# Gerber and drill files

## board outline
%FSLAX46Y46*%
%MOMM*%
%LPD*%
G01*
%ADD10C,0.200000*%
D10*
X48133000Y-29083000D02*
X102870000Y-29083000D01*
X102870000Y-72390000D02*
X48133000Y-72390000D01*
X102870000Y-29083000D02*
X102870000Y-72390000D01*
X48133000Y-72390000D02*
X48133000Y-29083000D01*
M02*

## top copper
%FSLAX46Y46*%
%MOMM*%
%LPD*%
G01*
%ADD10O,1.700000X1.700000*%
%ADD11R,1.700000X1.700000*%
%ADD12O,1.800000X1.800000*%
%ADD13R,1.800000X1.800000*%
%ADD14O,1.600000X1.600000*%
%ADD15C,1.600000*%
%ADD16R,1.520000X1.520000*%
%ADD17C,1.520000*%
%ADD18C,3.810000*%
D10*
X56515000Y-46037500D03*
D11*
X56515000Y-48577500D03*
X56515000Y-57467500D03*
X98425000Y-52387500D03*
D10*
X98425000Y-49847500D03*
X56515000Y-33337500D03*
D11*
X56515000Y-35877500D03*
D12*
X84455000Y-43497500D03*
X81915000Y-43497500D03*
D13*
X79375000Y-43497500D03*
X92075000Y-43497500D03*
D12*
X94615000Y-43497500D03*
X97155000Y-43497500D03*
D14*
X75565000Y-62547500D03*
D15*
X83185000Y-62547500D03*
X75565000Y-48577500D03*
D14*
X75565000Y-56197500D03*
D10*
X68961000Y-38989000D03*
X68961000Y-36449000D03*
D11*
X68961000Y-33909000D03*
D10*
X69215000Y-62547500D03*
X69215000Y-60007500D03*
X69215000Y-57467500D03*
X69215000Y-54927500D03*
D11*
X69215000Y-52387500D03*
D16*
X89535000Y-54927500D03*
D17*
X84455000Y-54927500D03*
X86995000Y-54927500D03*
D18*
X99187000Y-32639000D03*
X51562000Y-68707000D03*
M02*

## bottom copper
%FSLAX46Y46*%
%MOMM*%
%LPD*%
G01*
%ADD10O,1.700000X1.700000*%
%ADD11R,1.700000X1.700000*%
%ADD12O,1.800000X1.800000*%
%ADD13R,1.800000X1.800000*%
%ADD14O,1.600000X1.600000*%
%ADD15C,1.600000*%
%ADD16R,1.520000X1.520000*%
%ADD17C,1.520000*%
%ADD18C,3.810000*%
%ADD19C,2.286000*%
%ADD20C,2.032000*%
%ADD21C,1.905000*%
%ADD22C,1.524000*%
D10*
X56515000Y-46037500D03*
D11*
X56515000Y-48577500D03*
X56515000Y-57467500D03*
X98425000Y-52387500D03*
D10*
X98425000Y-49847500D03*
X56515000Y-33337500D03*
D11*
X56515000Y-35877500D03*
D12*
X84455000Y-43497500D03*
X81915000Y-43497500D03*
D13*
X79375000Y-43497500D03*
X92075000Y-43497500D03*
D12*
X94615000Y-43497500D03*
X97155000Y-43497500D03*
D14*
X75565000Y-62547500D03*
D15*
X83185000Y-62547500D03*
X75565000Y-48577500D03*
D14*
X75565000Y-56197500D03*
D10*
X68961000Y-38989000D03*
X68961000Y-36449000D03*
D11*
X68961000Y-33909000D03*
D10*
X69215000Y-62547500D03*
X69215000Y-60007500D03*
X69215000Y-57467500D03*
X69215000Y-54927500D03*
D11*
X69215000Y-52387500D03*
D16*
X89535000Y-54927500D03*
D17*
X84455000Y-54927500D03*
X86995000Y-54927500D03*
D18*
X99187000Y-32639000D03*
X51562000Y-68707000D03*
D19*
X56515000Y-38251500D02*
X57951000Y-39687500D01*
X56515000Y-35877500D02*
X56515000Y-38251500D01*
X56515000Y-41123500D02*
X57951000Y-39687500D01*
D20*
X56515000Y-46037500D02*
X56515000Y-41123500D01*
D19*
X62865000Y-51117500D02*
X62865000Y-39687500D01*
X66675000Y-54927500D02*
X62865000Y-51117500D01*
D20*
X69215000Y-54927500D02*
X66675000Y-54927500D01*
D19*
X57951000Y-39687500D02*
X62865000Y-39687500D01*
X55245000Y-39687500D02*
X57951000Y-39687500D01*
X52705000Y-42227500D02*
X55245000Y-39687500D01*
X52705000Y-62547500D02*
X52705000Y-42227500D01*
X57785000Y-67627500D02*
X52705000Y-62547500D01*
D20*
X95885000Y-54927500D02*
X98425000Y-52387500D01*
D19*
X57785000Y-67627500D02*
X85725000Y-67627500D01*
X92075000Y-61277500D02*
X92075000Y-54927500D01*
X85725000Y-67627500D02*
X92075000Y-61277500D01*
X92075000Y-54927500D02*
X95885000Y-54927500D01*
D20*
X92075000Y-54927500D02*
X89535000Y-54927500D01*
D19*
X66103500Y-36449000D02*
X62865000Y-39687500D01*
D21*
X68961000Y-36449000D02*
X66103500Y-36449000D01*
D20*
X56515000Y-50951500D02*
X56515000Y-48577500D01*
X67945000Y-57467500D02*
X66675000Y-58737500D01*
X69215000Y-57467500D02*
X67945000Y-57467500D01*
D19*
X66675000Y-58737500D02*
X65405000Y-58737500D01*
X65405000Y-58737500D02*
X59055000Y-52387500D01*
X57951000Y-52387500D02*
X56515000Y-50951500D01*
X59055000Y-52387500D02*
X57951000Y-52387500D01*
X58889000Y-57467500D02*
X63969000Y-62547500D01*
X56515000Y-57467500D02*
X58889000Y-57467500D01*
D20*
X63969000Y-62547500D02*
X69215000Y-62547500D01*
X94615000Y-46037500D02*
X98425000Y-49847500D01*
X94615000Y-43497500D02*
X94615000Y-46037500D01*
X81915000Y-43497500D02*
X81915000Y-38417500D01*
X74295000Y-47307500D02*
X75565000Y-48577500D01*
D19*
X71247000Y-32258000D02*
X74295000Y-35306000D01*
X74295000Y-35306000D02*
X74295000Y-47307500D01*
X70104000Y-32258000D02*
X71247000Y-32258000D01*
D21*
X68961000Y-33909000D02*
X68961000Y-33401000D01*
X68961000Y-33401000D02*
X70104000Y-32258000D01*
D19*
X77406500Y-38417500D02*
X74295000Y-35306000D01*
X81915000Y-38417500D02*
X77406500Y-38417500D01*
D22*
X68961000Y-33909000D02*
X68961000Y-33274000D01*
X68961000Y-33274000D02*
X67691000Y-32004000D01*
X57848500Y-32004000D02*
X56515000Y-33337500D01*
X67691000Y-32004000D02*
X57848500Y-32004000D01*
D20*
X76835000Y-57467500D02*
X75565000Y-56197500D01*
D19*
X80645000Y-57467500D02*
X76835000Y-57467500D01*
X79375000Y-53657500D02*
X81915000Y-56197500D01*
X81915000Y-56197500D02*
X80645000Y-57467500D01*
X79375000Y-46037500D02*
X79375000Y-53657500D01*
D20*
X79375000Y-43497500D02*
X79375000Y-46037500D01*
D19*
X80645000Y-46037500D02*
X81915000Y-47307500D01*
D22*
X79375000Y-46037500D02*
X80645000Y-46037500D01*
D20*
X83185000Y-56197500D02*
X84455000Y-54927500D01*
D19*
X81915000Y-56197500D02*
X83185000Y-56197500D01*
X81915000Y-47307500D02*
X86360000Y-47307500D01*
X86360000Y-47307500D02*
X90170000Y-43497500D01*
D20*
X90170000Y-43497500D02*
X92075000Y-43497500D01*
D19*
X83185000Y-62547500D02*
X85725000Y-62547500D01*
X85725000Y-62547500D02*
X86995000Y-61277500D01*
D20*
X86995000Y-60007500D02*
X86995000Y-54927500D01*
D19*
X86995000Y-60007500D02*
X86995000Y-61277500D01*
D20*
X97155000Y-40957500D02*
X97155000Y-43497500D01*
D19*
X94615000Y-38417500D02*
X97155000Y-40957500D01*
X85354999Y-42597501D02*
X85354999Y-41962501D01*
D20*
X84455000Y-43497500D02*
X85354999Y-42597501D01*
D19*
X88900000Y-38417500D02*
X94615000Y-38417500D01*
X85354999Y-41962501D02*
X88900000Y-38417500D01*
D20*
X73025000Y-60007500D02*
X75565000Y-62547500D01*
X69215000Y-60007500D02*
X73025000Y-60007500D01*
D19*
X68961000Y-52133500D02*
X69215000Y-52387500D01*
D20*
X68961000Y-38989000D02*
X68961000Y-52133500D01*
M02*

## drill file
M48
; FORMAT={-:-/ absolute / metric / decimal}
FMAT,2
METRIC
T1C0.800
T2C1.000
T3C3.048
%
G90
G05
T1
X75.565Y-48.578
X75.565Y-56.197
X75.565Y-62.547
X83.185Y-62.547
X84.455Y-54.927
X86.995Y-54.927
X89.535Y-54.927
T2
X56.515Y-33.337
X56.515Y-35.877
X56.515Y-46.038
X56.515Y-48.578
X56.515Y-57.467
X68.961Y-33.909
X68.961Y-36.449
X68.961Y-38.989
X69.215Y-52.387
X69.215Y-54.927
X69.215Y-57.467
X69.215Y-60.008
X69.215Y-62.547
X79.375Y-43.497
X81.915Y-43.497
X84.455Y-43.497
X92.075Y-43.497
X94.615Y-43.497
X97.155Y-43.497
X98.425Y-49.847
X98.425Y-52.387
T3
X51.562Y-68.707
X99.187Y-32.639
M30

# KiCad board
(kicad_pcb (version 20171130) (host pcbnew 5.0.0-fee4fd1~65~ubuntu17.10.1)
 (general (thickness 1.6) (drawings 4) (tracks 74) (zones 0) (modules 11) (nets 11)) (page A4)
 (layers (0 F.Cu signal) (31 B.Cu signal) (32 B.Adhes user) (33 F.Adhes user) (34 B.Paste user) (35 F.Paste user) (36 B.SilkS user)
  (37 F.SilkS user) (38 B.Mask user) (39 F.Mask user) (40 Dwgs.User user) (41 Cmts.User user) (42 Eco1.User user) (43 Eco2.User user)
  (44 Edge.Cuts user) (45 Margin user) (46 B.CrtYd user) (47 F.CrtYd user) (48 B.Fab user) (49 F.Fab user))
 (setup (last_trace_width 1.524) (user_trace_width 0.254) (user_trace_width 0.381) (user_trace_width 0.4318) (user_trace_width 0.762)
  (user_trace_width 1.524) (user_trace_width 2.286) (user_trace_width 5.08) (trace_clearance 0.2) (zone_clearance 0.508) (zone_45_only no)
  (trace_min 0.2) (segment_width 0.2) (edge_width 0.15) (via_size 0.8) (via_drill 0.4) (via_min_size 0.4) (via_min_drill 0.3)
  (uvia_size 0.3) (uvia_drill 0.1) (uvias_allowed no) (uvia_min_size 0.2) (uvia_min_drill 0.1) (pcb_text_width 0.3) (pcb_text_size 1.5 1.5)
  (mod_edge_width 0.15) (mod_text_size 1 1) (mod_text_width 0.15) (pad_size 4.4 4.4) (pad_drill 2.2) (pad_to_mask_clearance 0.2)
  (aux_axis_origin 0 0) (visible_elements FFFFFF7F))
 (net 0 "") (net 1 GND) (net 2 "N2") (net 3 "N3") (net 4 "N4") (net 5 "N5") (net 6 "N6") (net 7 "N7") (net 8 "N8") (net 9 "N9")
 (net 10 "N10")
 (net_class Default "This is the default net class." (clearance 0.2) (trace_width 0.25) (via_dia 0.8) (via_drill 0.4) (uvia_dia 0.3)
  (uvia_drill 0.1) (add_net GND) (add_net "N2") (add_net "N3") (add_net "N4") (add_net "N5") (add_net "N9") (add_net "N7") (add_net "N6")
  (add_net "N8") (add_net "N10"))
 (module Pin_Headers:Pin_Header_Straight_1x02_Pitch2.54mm (layer F.Cu) (at 56.515 48.5775 180)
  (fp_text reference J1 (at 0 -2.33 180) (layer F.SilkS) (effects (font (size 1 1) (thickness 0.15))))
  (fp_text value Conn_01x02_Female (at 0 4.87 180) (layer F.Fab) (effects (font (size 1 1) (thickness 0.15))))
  (pad 2 thru_hole oval (at 0 2.54 180) (size 1.7 1.7) (drill 1) (layers *.Cu *.Mask) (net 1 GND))
  (pad 1 thru_hole rect (at 0 0 180) (size 1.7 1.7) (drill 1) (layers *.Cu *.Mask) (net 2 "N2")))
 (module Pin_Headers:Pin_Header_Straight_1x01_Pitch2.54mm (layer F.Cu) (at 56.515 57.4675)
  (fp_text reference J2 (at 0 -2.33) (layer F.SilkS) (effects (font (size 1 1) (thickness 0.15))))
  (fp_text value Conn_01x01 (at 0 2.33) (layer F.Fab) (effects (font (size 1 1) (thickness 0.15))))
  (pad 1 thru_hole rect (at 0 0) (size 1.7 1.7) (drill 1) (layers *.Cu *.Mask) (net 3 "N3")))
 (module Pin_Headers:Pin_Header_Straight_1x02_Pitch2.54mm (layer F.Cu) (at 98.425 52.3875 180)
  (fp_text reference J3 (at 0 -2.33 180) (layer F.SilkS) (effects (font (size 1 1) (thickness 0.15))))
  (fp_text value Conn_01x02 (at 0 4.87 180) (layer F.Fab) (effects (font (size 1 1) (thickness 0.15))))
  (pad 1 thru_hole rect (at 0 0 180) (size 1.7 1.7) (drill 1) (layers *.Cu *.Mask) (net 1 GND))
  (pad 2 thru_hole oval (at 0 2.54 180) (size 1.7 1.7) (drill 1) (layers *.Cu *.Mask) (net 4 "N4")))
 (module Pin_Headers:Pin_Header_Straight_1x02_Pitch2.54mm (layer F.Cu) (at 56.515 35.8775 180)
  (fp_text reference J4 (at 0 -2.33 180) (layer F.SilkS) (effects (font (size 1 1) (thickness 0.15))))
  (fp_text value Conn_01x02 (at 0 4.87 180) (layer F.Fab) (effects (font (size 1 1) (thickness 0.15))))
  (pad 2 thru_hole oval (at 0 2.54 180) (size 1.7 1.7) (drill 1) (layers *.Cu *.Mask) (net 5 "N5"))
  (pad 1 thru_hole rect (at 0 0 180) (size 1.7 1.7) (drill 1) (layers *.Cu *.Mask) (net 1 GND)))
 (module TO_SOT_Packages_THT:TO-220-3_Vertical (layer F.Cu) (at 79.375 43.4975)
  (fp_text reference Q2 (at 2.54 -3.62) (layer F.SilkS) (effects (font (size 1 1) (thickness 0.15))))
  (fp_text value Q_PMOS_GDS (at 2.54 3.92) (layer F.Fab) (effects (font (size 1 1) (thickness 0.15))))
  (pad 3 thru_hole oval (at 5.08 0) (size 1.8 1.8) (drill 1) (layers *.Cu *.Mask) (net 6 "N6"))
  (pad 2 thru_hole oval (at 2.54 0) (size 1.8 1.8) (drill 1) (layers *.Cu *.Mask) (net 5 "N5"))
  (pad 1 thru_hole rect (at 0 0) (size 1.8 1.8) (drill 1) (layers *.Cu *.Mask) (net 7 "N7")))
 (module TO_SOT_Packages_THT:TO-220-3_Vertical (layer F.Cu) (at 92.075 43.4975)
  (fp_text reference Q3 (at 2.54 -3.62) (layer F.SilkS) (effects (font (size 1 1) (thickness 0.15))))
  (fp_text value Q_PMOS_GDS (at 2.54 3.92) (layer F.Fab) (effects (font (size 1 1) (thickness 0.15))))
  (pad 1 thru_hole rect (at 0 0) (size 1.8 1.8) (drill 1) (layers *.Cu *.Mask) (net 7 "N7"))
  (pad 2 thru_hole oval (at 2.54 0) (size 1.8 1.8) (drill 1) (layers *.Cu *.Mask) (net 4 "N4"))
  (pad 3 thru_hole oval (at 5.08 0) (size 1.8 1.8) (drill 1) (layers *.Cu *.Mask) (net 6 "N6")))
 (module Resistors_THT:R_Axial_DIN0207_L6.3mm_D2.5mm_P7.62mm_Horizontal (layer F.Cu) (at 83.185 62.5475 180)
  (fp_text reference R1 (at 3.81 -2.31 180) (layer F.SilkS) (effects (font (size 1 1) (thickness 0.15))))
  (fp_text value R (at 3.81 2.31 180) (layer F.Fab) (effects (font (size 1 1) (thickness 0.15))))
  (pad 2 thru_hole oval (at 7.62 0 180) (size 1.6 1.6) (drill 0.8) (layers *.Cu *.Mask) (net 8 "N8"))
  (pad 1 thru_hole circle (at 0 0 180) (size 1.6 1.6) (drill 0.8) (layers *.Cu *.Mask) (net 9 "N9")))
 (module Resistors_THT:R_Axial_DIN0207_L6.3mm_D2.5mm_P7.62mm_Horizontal (layer F.Cu) (at 75.565 48.5775 270)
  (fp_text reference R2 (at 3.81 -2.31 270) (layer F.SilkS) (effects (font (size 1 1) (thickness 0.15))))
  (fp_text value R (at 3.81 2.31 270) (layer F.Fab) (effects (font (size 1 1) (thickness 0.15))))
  (pad 1 thru_hole circle (at 0 0 270) (size 1.6 1.6) (drill 0.8) (layers *.Cu *.Mask) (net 5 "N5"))
  (pad 2 thru_hole oval (at 7.62 0 270) (size 1.6 1.6) (drill 0.8) (layers *.Cu *.Mask) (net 7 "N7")))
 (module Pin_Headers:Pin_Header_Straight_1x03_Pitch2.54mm (layer F.Cu) (at 68.961 33.909)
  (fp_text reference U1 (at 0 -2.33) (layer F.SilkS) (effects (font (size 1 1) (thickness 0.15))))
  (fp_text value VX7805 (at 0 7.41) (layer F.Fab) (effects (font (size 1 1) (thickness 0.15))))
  (pad 3 thru_hole oval (at 0 5.08) (size 1.7 1.7) (drill 1) (layers *.Cu *.Mask) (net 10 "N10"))
  (pad 2 thru_hole oval (at 0 2.54) (size 1.7 1.7) (drill 1) (layers *.Cu *.Mask) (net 1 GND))
  (pad 1 thru_hole rect (at 0 0) (size 1.7 1.7) (drill 1) (layers *.Cu *.Mask) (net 5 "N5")))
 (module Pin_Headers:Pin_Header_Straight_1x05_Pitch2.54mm (layer F.Cu) (at 69.215 52.3875)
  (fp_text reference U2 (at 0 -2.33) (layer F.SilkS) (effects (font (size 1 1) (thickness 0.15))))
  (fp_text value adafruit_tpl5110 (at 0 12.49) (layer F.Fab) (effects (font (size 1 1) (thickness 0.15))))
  (pad 5 thru_hole oval (at 0 10.16) (size 1.7 1.7) (drill 1) (layers *.Cu *.Mask) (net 3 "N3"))
  (pad 4 thru_hole oval (at 0 7.62) (size 1.7 1.7) (drill 1) (layers *.Cu *.Mask) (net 8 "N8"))
  (pad 3 thru_hole oval (at 0 5.08) (size 1.7 1.7) (drill 1) (layers *.Cu *.Mask) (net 2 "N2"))
  (pad 2 thru_hole oval (at 0 2.54) (size 1.7 1.7) (drill 1) (layers *.Cu *.Mask) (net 1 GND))
  (pad 1 thru_hole rect (at 0 0) (size 1.7 1.7) (drill 1) (layers *.Cu *.Mask) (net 10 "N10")))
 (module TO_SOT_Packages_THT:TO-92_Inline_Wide (layer F.Cu) (at 89.535 54.9275 180)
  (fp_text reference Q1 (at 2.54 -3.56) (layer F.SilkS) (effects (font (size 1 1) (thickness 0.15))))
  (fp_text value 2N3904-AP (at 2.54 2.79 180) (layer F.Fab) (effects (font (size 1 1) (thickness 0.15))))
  (pad 1 thru_hole rect (at 0 0 270) (size 1.52 1.52) (drill 0.8) (layers *.Cu *.Mask) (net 1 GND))
  (pad 3 thru_hole circle (at 5.08 0 270) (size 1.52 1.52) (drill 0.8) (layers *.Cu *.Mask) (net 7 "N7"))
  (pad 2 thru_hole circle (at 2.54 0 270) (size 1.52 1.52) (drill 0.8) (layers *.Cu *.Mask) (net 9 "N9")))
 (gr_line (start 48.133 29.083) (end 102.87 29.083) (layer Edge.Cuts) (width 0.2))
 (gr_line (start 102.87 72.39) (end 48.133 72.39) (layer Edge.Cuts) (width 0.2))
 (gr_line (start 102.87 29.083) (end 102.87 72.39) (layer Edge.Cuts) (width 0.2))
 (gr_line (start 48.133 72.39) (end 48.133 29.083) (layer Edge.Cuts) (width 0.2))
 (via (at 99.187 32.639) (size 3.81) (drill 3.048) (layers F.Cu B.Cu) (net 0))
 (via (at 51.562 68.707) (size 3.81) (drill 3.048) (layers F.Cu B.Cu) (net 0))
 (segment (start 56.515 38.2515) (end 57.951 39.6875) (width 2.286) (layer B.Cu) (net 1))
 (segment (start 56.515 35.8775) (end 56.515 38.2515) (width 2.286) (layer B.Cu) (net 1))
 (segment (start 56.515 41.1235) (end 57.951 39.6875) (width 2.286) (layer B.Cu) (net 1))
 (segment (start 56.515 46.0375) (end 56.515 41.1235) (width 2.032) (layer B.Cu) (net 1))
 (segment (start 62.865 51.1175) (end 62.865 39.6875) (width 2.286) (layer B.Cu) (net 1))
 (segment (start 66.675 54.9275) (end 62.865 51.1175) (width 2.286) (layer B.Cu) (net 1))
 (segment (start 69.215 54.9275) (end 66.675 54.9275) (width 2.032) (layer B.Cu) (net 1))
 (segment (start 57.951 39.6875) (end 62.865 39.6875) (width 2.286) (layer B.Cu) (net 1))
 (segment (start 55.245 39.6875) (end 57.951 39.6875) (width 2.286) (layer B.Cu) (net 1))
 (segment (start 52.705 42.2275) (end 55.245 39.6875) (width 2.286) (layer B.Cu) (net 1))
 (segment (start 52.705 62.5475) (end 52.705 42.2275) (width 2.286) (layer B.Cu) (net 1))
 (segment (start 57.785 67.6275) (end 52.705 62.5475) (width 2.286) (layer B.Cu) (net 1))
 (segment (start 95.885 54.9275) (end 98.425 52.3875) (width 2.032) (layer B.Cu) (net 1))
 (segment (start 57.785 67.6275) (end 85.725 67.6275) (width 2.286) (layer B.Cu) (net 1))
 (segment (start 92.075 61.2775) (end 92.075 54.9275) (width 2.286) (layer B.Cu) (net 1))
 (segment (start 85.725 67.6275) (end 92.075 61.2775) (width 2.286) (layer B.Cu) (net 1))
 (segment (start 92.075 54.9275) (end 95.885 54.9275) (width 2.286) (layer B.Cu) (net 1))
 (segment (start 92.075 54.9275) (end 89.535 54.9275) (width 2.032) (layer B.Cu) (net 1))
 (segment (start 66.1035 36.449) (end 62.865 39.6875) (width 2.286) (layer B.Cu) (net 1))
 (segment (start 68.961 36.449) (end 66.1035 36.449) (width 1.905) (layer B.Cu) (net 1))
 (segment (start 56.515 50.9515) (end 56.515 48.5775) (width 2.032) (layer B.Cu) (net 2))
 (segment (start 67.945 57.4675) (end 66.675 58.7375) (width 2.032) (layer B.Cu) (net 2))
 (segment (start 69.215 57.4675) (end 67.945 57.4675) (width 2.032) (layer B.Cu) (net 2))
 (segment (start 66.675 58.7375) (end 65.405 58.7375) (width 2.286) (layer B.Cu) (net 2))
 (segment (start 65.405 58.7375) (end 59.055 52.3875) (width 2.286) (layer B.Cu) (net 2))
 (segment (start 57.951 52.3875) (end 56.515 50.9515) (width 2.286) (layer B.Cu) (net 2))
 (segment (start 59.055 52.3875) (end 57.951 52.3875) (width 2.286) (layer B.Cu) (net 2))
 (segment (start 58.889 57.4675) (end 63.969 62.5475) (width 2.286) (layer B.Cu) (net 3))
 (segment (start 56.515 57.4675) (end 58.889 57.4675) (width 2.286) (layer B.Cu) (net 3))
 (segment (start 63.969 62.5475) (end 69.215 62.5475) (width 2.032) (layer B.Cu) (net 3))
 (segment (start 94.615 46.0375) (end 98.425 49.8475) (width 2.032) (layer B.Cu) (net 4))
 (segment (start 94.615 43.4975) (end 94.615 46.0375) (width 2.032) (layer B.Cu) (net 4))
 (segment (start 81.915 43.4975) (end 81.915 38.4175) (width 2.032) (layer B.Cu) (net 5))
 (segment (start 74.295 47.3075) (end 75.565 48.5775) (width 2.032) (layer B.Cu) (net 5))
 (segment (start 71.247 32.258) (end 74.295 35.306) (width 2.286) (layer B.Cu) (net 5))
 (segment (start 74.295 35.306) (end 74.295 47.3075) (width 2.286) (layer B.Cu) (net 5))
 (segment (start 70.104 32.258) (end 71.247 32.258) (width 2.286) (layer B.Cu) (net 5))
 (segment (start 68.961 33.909) (end 68.961 33.401) (width 1.905) (layer B.Cu) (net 5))
 (segment (start 68.961 33.401) (end 70.104 32.258) (width 1.905) (layer B.Cu) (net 5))
 (segment (start 77.4065 38.4175) (end 74.295 35.306) (width 2.286) (layer B.Cu) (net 5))
 (segment (start 81.915 38.4175) (end 77.4065 38.4175) (width 2.286) (layer B.Cu) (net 5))
 (segment (start 68.961 33.909) (end 68.961 33.274) (width 1.524) (layer B.Cu) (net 5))
 (segment (start 68.961 33.274) (end 67.691 32.004) (width 1.524) (layer B.Cu) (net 5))
 (segment (start 57.8485 32.004) (end 56.515 33.3375) (width 1.524) (layer B.Cu) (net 5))
 (segment (start 67.691 32.004) (end 57.8485 32.004) (width 1.524) (layer B.Cu) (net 5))
 (segment (start 76.835 57.4675) (end 75.565 56.1975) (width 2.032) (layer B.Cu) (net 7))
 (segment (start 80.645 57.4675) (end 76.835 57.4675) (width 2.286) (layer B.Cu) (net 7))
 (segment (start 79.375 53.6575) (end 81.915 56.1975) (width 2.286) (layer B.Cu) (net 7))
 (segment (start 81.915 56.1975) (end 80.645 57.4675) (width 2.286) (layer B.Cu) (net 7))
 (segment (start 79.375 46.0375) (end 79.375 53.6575) (width 2.286) (layer B.Cu) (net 7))
 (segment (start 79.375 43.4975) (end 79.375 46.0375) (width 2.032) (layer B.Cu) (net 7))
 (segment (start 80.645 46.0375) (end 81.915 47.3075) (width 2.286) (layer B.Cu) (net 7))
 (segment (start 79.375 46.0375) (end 80.645 46.0375) (width 1.524) (layer B.Cu) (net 7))
 (segment (start 83.185 56.1975) (end 84.455 54.9275) (width 2.032) (layer B.Cu) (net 7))
 (segment (start 81.915 56.1975) (end 83.185 56.1975) (width 2.286) (layer B.Cu) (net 7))
 (segment (start 81.915 47.3075) (end 86.36 47.3075) (width 2.286) (layer B.Cu) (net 7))
 (segment (start 86.36 47.3075) (end 90.17 43.4975) (width 2.286) (layer B.Cu) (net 7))
 (segment (start 90.17 43.4975) (end 92.075 43.4975) (width 2.032) (layer B.Cu) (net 7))
 (segment (start 83.185 62.5475) (end 85.725 62.5475) (width 2.286) (layer B.Cu) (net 9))
 (segment (start 85.725 62.5475) (end 86.995 61.2775) (width 2.286) (layer B.Cu) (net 9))
 (segment (start 86.995 60.0075) (end 86.995 54.9275) (width 2.032) (layer B.Cu) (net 9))
 (segment (start 86.995 60.0075) (end 86.995 61.2775) (width 2.286) (layer B.Cu) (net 9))
 (segment (start 97.155 40.9575) (end 97.155 43.4975) (width 2.032) (layer B.Cu) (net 6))
 (segment (start 94.615 38.4175) (end 97.155 40.9575) (width 2.286) (layer B.Cu) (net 6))
 (segment (start 85.354999 42.597501) (end 85.354999 41.962501) (width 2.286) (layer B.Cu) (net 6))
 (segment (start 84.455 43.4975) (end 85.354999 42.597501) (width 2.032) (layer B.Cu) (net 6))
 (segment (start 88.9 38.4175) (end 94.615 38.4175) (width 2.286) (layer B.Cu) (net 6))
 (segment (start 85.354999 41.962501) (end 88.9 38.4175) (width 2.286) (layer B.Cu) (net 6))
 (segment (start 73.025 60.0075) (end 75.565 62.5475) (width 2.032) (layer B.Cu) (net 8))
 (segment (start 69.215 60.0075) (end 73.025 60.0075) (width 2.032) (layer B.Cu) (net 8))
 (segment (start 68.961 52.1335) (end 69.215 52.3875) (width 2.286) (layer B.Cu) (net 10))
 (segment (start 68.961 38.989) (end 68.961 52.1335) (width 2.032) (layer B.Cu) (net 10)))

